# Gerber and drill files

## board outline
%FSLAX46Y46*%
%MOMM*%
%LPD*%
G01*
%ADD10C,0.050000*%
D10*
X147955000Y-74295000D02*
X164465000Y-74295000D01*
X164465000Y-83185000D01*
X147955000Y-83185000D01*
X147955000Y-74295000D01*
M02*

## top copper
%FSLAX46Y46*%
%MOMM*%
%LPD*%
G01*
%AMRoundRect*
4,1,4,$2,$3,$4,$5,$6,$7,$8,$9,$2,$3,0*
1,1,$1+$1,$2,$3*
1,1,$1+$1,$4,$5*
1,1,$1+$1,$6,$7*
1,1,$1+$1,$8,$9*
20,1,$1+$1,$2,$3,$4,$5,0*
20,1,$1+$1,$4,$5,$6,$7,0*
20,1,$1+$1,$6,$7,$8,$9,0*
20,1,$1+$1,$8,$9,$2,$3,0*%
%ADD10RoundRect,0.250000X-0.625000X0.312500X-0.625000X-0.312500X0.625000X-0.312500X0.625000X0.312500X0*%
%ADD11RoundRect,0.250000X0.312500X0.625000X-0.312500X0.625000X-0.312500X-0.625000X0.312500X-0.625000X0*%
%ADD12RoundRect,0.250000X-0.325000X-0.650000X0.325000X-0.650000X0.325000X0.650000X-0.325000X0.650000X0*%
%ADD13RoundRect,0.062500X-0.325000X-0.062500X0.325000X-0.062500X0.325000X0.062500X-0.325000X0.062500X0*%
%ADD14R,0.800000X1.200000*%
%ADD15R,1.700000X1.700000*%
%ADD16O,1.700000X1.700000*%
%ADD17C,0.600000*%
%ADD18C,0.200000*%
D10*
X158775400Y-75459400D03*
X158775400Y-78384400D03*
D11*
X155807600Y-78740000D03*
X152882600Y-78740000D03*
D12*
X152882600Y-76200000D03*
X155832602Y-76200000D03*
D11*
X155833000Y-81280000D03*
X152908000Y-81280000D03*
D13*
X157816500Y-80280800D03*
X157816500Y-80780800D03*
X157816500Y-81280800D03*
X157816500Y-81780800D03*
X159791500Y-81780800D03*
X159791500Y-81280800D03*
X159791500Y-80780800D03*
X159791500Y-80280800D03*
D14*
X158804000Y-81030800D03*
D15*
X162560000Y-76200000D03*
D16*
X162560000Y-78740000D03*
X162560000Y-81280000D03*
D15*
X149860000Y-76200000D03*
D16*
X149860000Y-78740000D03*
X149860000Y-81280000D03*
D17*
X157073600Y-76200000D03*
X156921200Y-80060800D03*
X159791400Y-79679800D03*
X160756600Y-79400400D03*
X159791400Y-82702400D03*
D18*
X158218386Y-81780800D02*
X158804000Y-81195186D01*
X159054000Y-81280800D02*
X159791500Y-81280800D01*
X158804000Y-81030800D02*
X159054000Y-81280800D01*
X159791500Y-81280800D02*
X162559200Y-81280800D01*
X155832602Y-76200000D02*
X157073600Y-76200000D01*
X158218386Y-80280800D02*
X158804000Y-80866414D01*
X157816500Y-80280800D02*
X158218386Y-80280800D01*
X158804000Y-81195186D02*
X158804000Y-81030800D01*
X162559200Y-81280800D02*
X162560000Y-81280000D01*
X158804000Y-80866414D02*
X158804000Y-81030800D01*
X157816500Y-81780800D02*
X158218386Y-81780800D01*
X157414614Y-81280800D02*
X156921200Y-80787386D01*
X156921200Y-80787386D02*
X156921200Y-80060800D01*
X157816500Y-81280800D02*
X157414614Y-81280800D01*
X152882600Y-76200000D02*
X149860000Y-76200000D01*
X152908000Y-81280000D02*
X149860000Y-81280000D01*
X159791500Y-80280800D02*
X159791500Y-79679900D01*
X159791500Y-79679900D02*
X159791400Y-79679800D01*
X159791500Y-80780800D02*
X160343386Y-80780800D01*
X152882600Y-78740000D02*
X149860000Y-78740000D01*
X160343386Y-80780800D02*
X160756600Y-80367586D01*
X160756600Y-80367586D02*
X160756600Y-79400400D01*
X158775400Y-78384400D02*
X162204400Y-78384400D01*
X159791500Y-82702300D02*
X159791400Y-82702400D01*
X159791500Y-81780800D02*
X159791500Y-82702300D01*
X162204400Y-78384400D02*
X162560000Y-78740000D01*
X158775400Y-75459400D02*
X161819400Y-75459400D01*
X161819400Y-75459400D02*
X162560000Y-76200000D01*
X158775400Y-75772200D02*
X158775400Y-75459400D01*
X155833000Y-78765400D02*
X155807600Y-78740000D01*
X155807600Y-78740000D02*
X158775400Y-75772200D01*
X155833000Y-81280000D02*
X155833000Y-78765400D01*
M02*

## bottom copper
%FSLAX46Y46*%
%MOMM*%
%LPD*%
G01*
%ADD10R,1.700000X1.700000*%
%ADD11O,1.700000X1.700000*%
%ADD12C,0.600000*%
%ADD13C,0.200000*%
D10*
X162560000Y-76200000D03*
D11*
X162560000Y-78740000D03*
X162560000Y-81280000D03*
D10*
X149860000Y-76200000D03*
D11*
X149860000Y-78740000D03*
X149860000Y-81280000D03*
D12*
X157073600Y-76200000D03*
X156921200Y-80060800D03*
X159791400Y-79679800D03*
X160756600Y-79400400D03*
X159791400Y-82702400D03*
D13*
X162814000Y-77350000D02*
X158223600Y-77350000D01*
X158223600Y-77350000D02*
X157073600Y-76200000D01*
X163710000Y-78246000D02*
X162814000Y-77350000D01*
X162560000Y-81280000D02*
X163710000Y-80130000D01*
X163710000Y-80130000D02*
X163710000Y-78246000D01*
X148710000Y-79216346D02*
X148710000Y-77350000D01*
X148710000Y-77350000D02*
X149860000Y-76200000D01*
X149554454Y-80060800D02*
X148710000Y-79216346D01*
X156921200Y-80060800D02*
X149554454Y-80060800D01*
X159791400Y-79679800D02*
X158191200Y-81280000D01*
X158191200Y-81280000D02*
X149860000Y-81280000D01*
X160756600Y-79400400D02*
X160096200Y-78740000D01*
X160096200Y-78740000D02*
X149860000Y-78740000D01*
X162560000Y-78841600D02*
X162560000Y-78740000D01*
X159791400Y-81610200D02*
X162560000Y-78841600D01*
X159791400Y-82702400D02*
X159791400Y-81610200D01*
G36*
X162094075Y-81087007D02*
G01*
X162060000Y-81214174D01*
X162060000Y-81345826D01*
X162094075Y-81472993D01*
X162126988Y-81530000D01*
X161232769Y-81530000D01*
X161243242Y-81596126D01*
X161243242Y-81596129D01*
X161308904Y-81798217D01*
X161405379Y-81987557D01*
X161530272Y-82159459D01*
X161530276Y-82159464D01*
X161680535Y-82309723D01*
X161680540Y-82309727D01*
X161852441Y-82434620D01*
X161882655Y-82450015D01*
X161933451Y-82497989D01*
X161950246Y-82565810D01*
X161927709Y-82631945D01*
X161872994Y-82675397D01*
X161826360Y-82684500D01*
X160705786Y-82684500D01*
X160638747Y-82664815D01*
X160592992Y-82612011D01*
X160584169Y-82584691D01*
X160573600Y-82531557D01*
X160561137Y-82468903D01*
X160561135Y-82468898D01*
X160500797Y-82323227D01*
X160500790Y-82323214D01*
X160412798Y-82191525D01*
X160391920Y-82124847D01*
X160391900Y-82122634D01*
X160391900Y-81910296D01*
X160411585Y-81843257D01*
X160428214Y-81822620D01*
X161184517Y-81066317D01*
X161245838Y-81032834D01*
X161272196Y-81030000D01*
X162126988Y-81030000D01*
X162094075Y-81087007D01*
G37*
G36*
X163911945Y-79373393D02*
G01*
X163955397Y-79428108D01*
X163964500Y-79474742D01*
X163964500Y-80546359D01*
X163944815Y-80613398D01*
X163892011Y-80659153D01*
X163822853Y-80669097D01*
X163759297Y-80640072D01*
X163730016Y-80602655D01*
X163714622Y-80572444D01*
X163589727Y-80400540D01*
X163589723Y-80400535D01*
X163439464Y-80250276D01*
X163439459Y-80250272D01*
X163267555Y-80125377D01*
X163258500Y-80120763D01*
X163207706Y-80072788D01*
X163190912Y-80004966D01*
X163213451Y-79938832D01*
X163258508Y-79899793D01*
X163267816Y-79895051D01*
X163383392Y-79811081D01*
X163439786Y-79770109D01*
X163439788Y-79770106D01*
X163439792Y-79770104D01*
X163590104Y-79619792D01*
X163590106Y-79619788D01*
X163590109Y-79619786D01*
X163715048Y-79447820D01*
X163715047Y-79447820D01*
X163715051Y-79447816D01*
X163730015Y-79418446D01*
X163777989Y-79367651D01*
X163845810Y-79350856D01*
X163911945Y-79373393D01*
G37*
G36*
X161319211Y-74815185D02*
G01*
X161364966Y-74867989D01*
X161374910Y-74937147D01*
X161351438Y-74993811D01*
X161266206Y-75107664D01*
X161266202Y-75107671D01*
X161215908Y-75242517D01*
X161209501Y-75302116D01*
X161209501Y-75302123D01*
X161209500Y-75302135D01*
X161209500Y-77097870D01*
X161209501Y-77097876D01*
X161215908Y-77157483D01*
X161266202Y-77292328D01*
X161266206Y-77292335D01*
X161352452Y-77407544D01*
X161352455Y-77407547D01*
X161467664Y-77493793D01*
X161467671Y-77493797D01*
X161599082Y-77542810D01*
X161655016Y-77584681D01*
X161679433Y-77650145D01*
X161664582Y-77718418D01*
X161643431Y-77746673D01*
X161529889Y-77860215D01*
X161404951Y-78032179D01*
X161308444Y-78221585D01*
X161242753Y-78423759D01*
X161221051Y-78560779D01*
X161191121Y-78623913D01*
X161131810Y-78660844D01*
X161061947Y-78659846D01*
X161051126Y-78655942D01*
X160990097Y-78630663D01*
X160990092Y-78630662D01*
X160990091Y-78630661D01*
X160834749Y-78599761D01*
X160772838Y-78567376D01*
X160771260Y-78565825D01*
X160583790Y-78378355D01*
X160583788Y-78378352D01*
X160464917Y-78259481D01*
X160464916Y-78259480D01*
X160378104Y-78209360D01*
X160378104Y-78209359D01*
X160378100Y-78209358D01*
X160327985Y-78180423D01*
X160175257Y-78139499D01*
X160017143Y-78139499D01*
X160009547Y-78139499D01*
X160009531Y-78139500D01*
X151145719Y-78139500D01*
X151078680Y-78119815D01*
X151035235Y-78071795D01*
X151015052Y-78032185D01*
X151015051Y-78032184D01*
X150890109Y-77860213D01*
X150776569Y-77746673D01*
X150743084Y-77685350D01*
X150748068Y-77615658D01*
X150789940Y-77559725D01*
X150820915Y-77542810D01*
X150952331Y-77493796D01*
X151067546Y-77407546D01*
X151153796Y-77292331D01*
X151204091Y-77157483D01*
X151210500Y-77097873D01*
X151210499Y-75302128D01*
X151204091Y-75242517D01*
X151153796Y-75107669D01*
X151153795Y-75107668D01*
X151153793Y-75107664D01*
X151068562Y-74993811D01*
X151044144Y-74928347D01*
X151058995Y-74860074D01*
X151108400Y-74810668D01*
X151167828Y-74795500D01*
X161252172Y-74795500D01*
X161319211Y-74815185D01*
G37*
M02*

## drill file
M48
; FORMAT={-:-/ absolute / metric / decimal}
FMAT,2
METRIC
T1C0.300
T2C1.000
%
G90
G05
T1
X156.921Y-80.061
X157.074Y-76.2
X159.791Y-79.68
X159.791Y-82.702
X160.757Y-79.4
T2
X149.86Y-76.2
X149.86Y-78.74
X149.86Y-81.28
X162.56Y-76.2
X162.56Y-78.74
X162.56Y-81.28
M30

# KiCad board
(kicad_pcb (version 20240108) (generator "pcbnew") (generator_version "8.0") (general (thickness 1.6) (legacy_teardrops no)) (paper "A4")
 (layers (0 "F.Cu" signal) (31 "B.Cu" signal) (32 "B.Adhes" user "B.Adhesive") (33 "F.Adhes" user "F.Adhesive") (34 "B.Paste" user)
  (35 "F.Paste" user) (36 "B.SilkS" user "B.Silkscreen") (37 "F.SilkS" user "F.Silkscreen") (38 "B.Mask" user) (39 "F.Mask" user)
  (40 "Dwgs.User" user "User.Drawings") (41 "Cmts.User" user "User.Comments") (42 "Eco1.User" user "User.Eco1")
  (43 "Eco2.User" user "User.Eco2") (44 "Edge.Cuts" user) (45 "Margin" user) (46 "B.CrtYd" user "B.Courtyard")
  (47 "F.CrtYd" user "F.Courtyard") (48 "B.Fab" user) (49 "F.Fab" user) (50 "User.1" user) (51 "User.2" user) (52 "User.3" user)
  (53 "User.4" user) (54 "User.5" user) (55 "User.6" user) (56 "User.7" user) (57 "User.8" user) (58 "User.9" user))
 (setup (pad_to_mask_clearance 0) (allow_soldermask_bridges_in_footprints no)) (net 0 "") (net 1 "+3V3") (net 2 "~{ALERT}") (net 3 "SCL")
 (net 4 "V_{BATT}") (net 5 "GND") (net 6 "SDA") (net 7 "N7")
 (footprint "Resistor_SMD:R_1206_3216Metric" (layer "F.Cu") (at 158.7754 76.9219 -90)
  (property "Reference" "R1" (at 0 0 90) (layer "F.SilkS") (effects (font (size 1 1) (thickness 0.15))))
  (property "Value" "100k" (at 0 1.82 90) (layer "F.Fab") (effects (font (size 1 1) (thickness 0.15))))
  (pad "1" smd roundrect (at -1.4625 0 270) (size 1.125 1.75) (layers "F.Cu" "F.Paste" "F.Mask") (roundrect_rratio 0.222222) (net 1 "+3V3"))
  (pad "2" smd roundrect (at 1.4625 0 270) (size 1.125 1.75) (layers "F.Cu" "F.Paste" "F.Mask") (roundrect_rratio 0.222222)
   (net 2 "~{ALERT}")))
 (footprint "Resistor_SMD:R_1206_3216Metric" (layer "F.Cu") (at 154.3451 78.74 180)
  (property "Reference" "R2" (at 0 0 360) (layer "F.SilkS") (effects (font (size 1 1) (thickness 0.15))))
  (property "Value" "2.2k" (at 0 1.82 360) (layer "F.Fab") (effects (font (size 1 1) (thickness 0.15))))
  (pad "1" smd roundrect (at -1.4625 0 180) (size 1.125 1.75) (layers "F.Cu" "F.Paste" "F.Mask") (roundrect_rratio 0.222222) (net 1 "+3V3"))
  (pad "2" smd roundrect (at 1.4625 0 180) (size 1.125 1.75) (layers "F.Cu" "F.Paste" "F.Mask") (roundrect_rratio 0.222222) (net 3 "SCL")))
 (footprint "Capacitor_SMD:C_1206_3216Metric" (layer "F.Cu") (at 154.357601 76.2)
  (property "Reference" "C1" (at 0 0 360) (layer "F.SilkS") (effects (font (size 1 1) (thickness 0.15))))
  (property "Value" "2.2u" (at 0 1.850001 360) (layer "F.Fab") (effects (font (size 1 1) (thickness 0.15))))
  (pad "1" smd roundrect (at -1.475001 0) (size 1.15 1.8) (layers "F.Cu" "F.Paste" "F.Mask") (roundrect_rratio 0.217391) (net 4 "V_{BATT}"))
  (pad "2" smd roundrect (at 1.475001 0) (size 1.15 1.8) (layers "F.Cu" "F.Paste" "F.Mask") (roundrect_rratio 0.217391) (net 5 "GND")))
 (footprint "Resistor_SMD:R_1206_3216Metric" (layer "F.Cu") (at 154.3705 81.28 180)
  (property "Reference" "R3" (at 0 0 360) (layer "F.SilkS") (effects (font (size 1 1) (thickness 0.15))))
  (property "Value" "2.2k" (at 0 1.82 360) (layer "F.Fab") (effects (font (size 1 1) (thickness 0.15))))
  (pad "1" smd roundrect (at -1.4625 0 180) (size 1.125 1.75) (layers "F.Cu" "F.Paste" "F.Mask") (roundrect_rratio 0.222222) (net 1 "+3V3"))
  (pad "2" smd roundrect (at 1.4625 0 180) (size 1.125 1.75) (layers "F.Cu" "F.Paste" "F.Mask") (roundrect_rratio 0.222222) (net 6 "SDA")))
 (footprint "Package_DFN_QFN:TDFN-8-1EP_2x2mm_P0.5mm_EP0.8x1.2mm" (layer "F.Cu") (at 158.804 81.0308)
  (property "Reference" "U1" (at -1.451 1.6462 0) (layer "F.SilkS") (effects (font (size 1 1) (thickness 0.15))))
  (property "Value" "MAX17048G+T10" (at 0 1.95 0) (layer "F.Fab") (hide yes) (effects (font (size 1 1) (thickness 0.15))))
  (pad "" smd roundrect (at -0.2 -0.3) (size 0.32 0.48) (layers "F.Paste") (roundrect_rratio 0.25))
  (pad "" smd roundrect (at -0.2 0.3) (size 0.32 0.48) (layers "F.Paste") (roundrect_rratio 0.25))
  (pad "" smd roundrect (at 0.2 -0.3) (size 0.32 0.48) (layers "F.Paste") (roundrect_rratio 0.25))
  (pad "" smd roundrect (at 0.2 0.3) (size 0.32 0.48) (layers "F.Paste") (roundrect_rratio 0.25))
  (pad "1" smd roundrect (at -0.9875 -0.75) (size 0.775 0.25) (layers "F.Cu" "F.Paste" "F.Mask") (roundrect_rratio 0.25) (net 5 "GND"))
  (pad "2" smd roundrect (at -0.9875 -0.25) (size 0.775 0.25) (layers "F.Cu" "F.Paste" "F.Mask") (roundrect_rratio 0.25) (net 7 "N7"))
  (pad "3" smd roundrect (at -0.9875 0.25) (size 0.775 0.25) (layers "F.Cu" "F.Paste" "F.Mask") (roundrect_rratio 0.25) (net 4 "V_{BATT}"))
  (pad "4" smd roundrect (at -0.9875 0.75) (size 0.775 0.25) (layers "F.Cu" "F.Paste" "F.Mask") (roundrect_rratio 0.25) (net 5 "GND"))
  (pad "5" smd roundrect (at 0.9875 0.75) (size 0.775 0.25) (layers "F.Cu" "F.Paste" "F.Mask") (roundrect_rratio 0.25) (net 2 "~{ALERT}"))
  (pad "6" smd roundrect (at 0.9875 0.25) (size 0.775 0.25) (layers "F.Cu" "F.Paste" "F.Mask") (roundrect_rratio 0.25) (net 5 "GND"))
  (pad "7" smd roundrect (at 0.9875 -0.25) (size 0.775 0.25) (layers "F.Cu" "F.Paste" "F.Mask") (roundrect_rratio 0.25) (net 3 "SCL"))
  (pad "8" smd roundrect (at 0.9875 -0.75) (size 0.775 0.25) (layers "F.Cu" "F.Paste" "F.Mask") (roundrect_rratio 0.25) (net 6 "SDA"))
  (pad "9" smd rect (at 0 0) (size 0.8 1.2) (layers "F.Cu" "F.Mask") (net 5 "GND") (zone_connect 2)))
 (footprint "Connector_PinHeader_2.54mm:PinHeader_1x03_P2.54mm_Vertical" (layer "B.Cu") (at 162.56 76.2 180)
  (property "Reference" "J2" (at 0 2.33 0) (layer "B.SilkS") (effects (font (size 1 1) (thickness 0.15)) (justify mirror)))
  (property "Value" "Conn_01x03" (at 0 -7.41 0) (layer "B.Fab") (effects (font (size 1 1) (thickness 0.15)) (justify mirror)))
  (pad "1" thru_hole rect (at 0 0 180) (size 1.7 1.7) (drill 1) (layers "*.Cu" "*.Mask") (remove_unused_layers no) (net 1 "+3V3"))
  (pad "2" thru_hole oval (at 0 -2.54 180) (size 1.7 1.7) (drill 1) (layers "*.Cu" "*.Mask") (remove_unused_layers no) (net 2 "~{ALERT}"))
  (pad "3" thru_hole oval (at 0 -5.08 180) (size 1.7 1.7) (drill 1) (layers "*.Cu" "*.Mask") (remove_unused_layers no) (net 5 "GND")))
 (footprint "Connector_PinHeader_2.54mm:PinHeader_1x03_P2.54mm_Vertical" (layer "B.Cu") (at 149.86 76.2 180)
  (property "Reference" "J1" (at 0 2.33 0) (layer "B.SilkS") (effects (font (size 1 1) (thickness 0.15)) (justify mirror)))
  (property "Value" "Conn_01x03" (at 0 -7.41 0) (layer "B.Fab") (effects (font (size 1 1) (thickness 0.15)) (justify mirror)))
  (pad "1" thru_hole rect (at 0 0 180) (size 1.7 1.7) (drill 1) (layers "*.Cu" "*.Mask") (remove_unused_layers no) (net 4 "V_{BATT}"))
  (pad "2" thru_hole oval (at 0 -2.54 180) (size 1.7 1.7) (drill 1) (layers "*.Cu" "*.Mask") (remove_unused_layers no) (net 3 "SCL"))
  (pad "3" thru_hole oval (at 0 -5.08 180) (size 1.7 1.7) (drill 1) (layers "*.Cu" "*.Mask") (remove_unused_layers no) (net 6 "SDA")))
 (gr_rect (start 147.955 74.295) (end 164.465 83.185) (stroke (width 0.05) (type default)) (fill none) (layer "Edge.Cuts"))
 (segment (start 158.218386 81.7808) (end 158.804 81.195186) (width 0.2) (layer "F.Cu") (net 5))
 (segment (start 159.054 81.2808) (end 159.7915 81.2808) (width 0.2) (layer "F.Cu") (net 5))
 (segment (start 158.804 81.0308) (end 159.054 81.2808) (width 0.2) (layer "F.Cu") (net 5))
 (segment (start 159.7915 81.2808) (end 162.5592 81.2808) (width 0.2) (layer "F.Cu") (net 5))
 (segment (start 155.832602 76.2) (end 157.0736 76.2) (width 0.2) (layer "F.Cu") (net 5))
 (segment (start 158.218386 80.2808) (end 158.804 80.866414) (width 0.2) (layer "F.Cu") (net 5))
 (segment (start 157.8165 80.2808) (end 158.218386 80.2808) (width 0.2) (layer "F.Cu") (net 5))
 (segment (start 158.804 81.195186) (end 158.804 81.0308) (width 0.2) (layer "F.Cu") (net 5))
 (segment (start 162.5592 81.2808) (end 162.56 81.28) (width 0.2) (layer "F.Cu") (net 5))
 (segment (start 158.804 80.866414) (end 158.804 81.0308) (width 0.2) (layer "F.Cu") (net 5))
 (segment (start 157.8165 81.7808) (end 158.218386 81.7808) (width 0.2) (layer "F.Cu") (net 5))
 (via (at 157.0736 76.2) (size 0.6) (drill 0.3) (layers "F.Cu" "B.Cu") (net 5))
 (segment (start 162.814 77.35) (end 158.2236 77.35) (width 0.2) (layer "B.Cu") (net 5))
 (segment (start 158.2236 77.35) (end 157.0736 76.2) (width 0.2) (layer "B.Cu") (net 5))
 (segment (start 163.71 78.246) (end 162.814 77.35) (width 0.2) (layer "B.Cu") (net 5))
 (segment (start 162.56 81.28) (end 163.71 80.13) (width 0.2) (layer "B.Cu") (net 5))
 (segment (start 163.71 80.13) (end 163.71 78.246) (width 0.2) (layer "B.Cu") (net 5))
 (segment (start 157.414614 81.2808) (end 156.9212 80.787386) (width 0.2) (layer "F.Cu") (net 4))
 (segment (start 156.9212 80.787386) (end 156.9212 80.0608) (width 0.2) (layer "F.Cu") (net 4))
 (segment (start 157.8165 81.2808) (end 157.414614 81.2808) (width 0.2) (layer "F.Cu") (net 4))
 (segment (start 152.8826 76.2) (end 149.86 76.2) (width 0.2) (layer "F.Cu") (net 4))
 (via (at 156.9212 80.0608) (size 0.6) (drill 0.3) (layers "F.Cu" "B.Cu") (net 4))
 (segment (start 148.71 79.216346) (end 148.71 77.35) (width 0.2) (layer "B.Cu") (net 4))
 (segment (start 148.71 77.35) (end 149.86 76.2) (width 0.2) (layer "B.Cu") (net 4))
 (segment (start 149.554454 80.0608) (end 148.71 79.216346) (width 0.2) (layer "B.Cu") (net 4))
 (segment (start 156.9212 80.0608) (end 149.554454 80.0608) (width 0.2) (layer "B.Cu") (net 4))
 (segment (start 152.908 81.28) (end 149.86 81.28) (width 0.2) (layer "F.Cu") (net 6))
 (segment (start 159.7915 80.2808) (end 159.7915 79.6799) (width 0.2) (layer "F.Cu") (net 6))
 (segment (start 159.7915 79.6799) (end 159.7914 79.6798) (width 0.2) (layer "F.Cu") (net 6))
 (via (at 159.7914 79.6798) (size 0.6) (drill 0.3) (layers "F.Cu" "B.Cu") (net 6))
 (segment (start 159.7914 79.6798) (end 158.1912 81.28) (width 0.2) (layer "B.Cu") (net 6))
 (segment (start 158.1912 81.28) (end 149.86 81.28) (width 0.2) (layer "B.Cu") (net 6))
 (segment (start 159.7915 80.7808) (end 160.343386 80.7808) (width 0.2) (layer "F.Cu") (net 3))
 (segment (start 152.8826 78.74) (end 149.86 78.74) (width 0.2) (layer "F.Cu") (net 3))
 (segment (start 160.343386 80.7808) (end 160.7566 80.367586) (width 0.2) (layer "F.Cu") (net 3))
 (segment (start 160.7566 80.367586) (end 160.7566 79.4004) (width 0.2) (layer "F.Cu") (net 3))
 (via (at 160.7566 79.4004) (size 0.6) (drill 0.3) (layers "F.Cu" "B.Cu") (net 3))
 (segment (start 160.7566 79.4004) (end 160.0962 78.74) (width 0.2) (layer "B.Cu") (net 3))
 (segment (start 160.0962 78.74) (end 149.86 78.74) (width 0.2) (layer "B.Cu") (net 3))
 (segment (start 158.7754 78.3844) (end 162.2044 78.3844) (width 0.2) (layer "F.Cu") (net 2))
 (segment (start 159.7915 82.7023) (end 159.7914 82.7024) (width 0.2) (layer "F.Cu") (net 2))
 (segment (start 159.7915 81.7808) (end 159.7915 82.7023) (width 0.2) (layer "F.Cu") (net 2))
 (segment (start 162.2044 78.3844) (end 162.56 78.74) (width 0.2) (layer "F.Cu") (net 2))
 (via (at 159.7914 82.7024) (size 0.6) (drill 0.3) (layers "F.Cu" "B.Cu") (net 2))
 (segment (start 162.56 78.8416) (end 162.56 78.74) (width 0.2) (layer "B.Cu") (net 2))
 (segment (start 159.7914 81.6102) (end 162.56 78.8416) (width 0.2) (layer "B.Cu") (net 2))
 (segment (start 159.7914 82.7024) (end 159.7914 81.6102) (width 0.2) (layer "B.Cu") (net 2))
 (segment (start 158.7754 75.4594) (end 161.8194 75.4594) (width 0.2) (layer "F.Cu") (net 1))
 (segment (start 161.8194 75.4594) (end 162.56 76.2) (width 0.2) (layer "F.Cu") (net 1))
 (segment (start 158.7754 75.7722) (end 158.7754 75.4594) (width 0.2) (layer "F.Cu") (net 1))
 (segment (start 155.833 78.7654) (end 155.8076 78.74) (width 0.2) (layer "F.Cu") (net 1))
 (segment (start 155.8076 78.74) (end 158.7754 75.7722) (width 0.2) (layer "F.Cu") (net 1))
 (segment (start 155.833 81.28) (end 155.833 78.7654) (width 0.2) (layer "F.Cu") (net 1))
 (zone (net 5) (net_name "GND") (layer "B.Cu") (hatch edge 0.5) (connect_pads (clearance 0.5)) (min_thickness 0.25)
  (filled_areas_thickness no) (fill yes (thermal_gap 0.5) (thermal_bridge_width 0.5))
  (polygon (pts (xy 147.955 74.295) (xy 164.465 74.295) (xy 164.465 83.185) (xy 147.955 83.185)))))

